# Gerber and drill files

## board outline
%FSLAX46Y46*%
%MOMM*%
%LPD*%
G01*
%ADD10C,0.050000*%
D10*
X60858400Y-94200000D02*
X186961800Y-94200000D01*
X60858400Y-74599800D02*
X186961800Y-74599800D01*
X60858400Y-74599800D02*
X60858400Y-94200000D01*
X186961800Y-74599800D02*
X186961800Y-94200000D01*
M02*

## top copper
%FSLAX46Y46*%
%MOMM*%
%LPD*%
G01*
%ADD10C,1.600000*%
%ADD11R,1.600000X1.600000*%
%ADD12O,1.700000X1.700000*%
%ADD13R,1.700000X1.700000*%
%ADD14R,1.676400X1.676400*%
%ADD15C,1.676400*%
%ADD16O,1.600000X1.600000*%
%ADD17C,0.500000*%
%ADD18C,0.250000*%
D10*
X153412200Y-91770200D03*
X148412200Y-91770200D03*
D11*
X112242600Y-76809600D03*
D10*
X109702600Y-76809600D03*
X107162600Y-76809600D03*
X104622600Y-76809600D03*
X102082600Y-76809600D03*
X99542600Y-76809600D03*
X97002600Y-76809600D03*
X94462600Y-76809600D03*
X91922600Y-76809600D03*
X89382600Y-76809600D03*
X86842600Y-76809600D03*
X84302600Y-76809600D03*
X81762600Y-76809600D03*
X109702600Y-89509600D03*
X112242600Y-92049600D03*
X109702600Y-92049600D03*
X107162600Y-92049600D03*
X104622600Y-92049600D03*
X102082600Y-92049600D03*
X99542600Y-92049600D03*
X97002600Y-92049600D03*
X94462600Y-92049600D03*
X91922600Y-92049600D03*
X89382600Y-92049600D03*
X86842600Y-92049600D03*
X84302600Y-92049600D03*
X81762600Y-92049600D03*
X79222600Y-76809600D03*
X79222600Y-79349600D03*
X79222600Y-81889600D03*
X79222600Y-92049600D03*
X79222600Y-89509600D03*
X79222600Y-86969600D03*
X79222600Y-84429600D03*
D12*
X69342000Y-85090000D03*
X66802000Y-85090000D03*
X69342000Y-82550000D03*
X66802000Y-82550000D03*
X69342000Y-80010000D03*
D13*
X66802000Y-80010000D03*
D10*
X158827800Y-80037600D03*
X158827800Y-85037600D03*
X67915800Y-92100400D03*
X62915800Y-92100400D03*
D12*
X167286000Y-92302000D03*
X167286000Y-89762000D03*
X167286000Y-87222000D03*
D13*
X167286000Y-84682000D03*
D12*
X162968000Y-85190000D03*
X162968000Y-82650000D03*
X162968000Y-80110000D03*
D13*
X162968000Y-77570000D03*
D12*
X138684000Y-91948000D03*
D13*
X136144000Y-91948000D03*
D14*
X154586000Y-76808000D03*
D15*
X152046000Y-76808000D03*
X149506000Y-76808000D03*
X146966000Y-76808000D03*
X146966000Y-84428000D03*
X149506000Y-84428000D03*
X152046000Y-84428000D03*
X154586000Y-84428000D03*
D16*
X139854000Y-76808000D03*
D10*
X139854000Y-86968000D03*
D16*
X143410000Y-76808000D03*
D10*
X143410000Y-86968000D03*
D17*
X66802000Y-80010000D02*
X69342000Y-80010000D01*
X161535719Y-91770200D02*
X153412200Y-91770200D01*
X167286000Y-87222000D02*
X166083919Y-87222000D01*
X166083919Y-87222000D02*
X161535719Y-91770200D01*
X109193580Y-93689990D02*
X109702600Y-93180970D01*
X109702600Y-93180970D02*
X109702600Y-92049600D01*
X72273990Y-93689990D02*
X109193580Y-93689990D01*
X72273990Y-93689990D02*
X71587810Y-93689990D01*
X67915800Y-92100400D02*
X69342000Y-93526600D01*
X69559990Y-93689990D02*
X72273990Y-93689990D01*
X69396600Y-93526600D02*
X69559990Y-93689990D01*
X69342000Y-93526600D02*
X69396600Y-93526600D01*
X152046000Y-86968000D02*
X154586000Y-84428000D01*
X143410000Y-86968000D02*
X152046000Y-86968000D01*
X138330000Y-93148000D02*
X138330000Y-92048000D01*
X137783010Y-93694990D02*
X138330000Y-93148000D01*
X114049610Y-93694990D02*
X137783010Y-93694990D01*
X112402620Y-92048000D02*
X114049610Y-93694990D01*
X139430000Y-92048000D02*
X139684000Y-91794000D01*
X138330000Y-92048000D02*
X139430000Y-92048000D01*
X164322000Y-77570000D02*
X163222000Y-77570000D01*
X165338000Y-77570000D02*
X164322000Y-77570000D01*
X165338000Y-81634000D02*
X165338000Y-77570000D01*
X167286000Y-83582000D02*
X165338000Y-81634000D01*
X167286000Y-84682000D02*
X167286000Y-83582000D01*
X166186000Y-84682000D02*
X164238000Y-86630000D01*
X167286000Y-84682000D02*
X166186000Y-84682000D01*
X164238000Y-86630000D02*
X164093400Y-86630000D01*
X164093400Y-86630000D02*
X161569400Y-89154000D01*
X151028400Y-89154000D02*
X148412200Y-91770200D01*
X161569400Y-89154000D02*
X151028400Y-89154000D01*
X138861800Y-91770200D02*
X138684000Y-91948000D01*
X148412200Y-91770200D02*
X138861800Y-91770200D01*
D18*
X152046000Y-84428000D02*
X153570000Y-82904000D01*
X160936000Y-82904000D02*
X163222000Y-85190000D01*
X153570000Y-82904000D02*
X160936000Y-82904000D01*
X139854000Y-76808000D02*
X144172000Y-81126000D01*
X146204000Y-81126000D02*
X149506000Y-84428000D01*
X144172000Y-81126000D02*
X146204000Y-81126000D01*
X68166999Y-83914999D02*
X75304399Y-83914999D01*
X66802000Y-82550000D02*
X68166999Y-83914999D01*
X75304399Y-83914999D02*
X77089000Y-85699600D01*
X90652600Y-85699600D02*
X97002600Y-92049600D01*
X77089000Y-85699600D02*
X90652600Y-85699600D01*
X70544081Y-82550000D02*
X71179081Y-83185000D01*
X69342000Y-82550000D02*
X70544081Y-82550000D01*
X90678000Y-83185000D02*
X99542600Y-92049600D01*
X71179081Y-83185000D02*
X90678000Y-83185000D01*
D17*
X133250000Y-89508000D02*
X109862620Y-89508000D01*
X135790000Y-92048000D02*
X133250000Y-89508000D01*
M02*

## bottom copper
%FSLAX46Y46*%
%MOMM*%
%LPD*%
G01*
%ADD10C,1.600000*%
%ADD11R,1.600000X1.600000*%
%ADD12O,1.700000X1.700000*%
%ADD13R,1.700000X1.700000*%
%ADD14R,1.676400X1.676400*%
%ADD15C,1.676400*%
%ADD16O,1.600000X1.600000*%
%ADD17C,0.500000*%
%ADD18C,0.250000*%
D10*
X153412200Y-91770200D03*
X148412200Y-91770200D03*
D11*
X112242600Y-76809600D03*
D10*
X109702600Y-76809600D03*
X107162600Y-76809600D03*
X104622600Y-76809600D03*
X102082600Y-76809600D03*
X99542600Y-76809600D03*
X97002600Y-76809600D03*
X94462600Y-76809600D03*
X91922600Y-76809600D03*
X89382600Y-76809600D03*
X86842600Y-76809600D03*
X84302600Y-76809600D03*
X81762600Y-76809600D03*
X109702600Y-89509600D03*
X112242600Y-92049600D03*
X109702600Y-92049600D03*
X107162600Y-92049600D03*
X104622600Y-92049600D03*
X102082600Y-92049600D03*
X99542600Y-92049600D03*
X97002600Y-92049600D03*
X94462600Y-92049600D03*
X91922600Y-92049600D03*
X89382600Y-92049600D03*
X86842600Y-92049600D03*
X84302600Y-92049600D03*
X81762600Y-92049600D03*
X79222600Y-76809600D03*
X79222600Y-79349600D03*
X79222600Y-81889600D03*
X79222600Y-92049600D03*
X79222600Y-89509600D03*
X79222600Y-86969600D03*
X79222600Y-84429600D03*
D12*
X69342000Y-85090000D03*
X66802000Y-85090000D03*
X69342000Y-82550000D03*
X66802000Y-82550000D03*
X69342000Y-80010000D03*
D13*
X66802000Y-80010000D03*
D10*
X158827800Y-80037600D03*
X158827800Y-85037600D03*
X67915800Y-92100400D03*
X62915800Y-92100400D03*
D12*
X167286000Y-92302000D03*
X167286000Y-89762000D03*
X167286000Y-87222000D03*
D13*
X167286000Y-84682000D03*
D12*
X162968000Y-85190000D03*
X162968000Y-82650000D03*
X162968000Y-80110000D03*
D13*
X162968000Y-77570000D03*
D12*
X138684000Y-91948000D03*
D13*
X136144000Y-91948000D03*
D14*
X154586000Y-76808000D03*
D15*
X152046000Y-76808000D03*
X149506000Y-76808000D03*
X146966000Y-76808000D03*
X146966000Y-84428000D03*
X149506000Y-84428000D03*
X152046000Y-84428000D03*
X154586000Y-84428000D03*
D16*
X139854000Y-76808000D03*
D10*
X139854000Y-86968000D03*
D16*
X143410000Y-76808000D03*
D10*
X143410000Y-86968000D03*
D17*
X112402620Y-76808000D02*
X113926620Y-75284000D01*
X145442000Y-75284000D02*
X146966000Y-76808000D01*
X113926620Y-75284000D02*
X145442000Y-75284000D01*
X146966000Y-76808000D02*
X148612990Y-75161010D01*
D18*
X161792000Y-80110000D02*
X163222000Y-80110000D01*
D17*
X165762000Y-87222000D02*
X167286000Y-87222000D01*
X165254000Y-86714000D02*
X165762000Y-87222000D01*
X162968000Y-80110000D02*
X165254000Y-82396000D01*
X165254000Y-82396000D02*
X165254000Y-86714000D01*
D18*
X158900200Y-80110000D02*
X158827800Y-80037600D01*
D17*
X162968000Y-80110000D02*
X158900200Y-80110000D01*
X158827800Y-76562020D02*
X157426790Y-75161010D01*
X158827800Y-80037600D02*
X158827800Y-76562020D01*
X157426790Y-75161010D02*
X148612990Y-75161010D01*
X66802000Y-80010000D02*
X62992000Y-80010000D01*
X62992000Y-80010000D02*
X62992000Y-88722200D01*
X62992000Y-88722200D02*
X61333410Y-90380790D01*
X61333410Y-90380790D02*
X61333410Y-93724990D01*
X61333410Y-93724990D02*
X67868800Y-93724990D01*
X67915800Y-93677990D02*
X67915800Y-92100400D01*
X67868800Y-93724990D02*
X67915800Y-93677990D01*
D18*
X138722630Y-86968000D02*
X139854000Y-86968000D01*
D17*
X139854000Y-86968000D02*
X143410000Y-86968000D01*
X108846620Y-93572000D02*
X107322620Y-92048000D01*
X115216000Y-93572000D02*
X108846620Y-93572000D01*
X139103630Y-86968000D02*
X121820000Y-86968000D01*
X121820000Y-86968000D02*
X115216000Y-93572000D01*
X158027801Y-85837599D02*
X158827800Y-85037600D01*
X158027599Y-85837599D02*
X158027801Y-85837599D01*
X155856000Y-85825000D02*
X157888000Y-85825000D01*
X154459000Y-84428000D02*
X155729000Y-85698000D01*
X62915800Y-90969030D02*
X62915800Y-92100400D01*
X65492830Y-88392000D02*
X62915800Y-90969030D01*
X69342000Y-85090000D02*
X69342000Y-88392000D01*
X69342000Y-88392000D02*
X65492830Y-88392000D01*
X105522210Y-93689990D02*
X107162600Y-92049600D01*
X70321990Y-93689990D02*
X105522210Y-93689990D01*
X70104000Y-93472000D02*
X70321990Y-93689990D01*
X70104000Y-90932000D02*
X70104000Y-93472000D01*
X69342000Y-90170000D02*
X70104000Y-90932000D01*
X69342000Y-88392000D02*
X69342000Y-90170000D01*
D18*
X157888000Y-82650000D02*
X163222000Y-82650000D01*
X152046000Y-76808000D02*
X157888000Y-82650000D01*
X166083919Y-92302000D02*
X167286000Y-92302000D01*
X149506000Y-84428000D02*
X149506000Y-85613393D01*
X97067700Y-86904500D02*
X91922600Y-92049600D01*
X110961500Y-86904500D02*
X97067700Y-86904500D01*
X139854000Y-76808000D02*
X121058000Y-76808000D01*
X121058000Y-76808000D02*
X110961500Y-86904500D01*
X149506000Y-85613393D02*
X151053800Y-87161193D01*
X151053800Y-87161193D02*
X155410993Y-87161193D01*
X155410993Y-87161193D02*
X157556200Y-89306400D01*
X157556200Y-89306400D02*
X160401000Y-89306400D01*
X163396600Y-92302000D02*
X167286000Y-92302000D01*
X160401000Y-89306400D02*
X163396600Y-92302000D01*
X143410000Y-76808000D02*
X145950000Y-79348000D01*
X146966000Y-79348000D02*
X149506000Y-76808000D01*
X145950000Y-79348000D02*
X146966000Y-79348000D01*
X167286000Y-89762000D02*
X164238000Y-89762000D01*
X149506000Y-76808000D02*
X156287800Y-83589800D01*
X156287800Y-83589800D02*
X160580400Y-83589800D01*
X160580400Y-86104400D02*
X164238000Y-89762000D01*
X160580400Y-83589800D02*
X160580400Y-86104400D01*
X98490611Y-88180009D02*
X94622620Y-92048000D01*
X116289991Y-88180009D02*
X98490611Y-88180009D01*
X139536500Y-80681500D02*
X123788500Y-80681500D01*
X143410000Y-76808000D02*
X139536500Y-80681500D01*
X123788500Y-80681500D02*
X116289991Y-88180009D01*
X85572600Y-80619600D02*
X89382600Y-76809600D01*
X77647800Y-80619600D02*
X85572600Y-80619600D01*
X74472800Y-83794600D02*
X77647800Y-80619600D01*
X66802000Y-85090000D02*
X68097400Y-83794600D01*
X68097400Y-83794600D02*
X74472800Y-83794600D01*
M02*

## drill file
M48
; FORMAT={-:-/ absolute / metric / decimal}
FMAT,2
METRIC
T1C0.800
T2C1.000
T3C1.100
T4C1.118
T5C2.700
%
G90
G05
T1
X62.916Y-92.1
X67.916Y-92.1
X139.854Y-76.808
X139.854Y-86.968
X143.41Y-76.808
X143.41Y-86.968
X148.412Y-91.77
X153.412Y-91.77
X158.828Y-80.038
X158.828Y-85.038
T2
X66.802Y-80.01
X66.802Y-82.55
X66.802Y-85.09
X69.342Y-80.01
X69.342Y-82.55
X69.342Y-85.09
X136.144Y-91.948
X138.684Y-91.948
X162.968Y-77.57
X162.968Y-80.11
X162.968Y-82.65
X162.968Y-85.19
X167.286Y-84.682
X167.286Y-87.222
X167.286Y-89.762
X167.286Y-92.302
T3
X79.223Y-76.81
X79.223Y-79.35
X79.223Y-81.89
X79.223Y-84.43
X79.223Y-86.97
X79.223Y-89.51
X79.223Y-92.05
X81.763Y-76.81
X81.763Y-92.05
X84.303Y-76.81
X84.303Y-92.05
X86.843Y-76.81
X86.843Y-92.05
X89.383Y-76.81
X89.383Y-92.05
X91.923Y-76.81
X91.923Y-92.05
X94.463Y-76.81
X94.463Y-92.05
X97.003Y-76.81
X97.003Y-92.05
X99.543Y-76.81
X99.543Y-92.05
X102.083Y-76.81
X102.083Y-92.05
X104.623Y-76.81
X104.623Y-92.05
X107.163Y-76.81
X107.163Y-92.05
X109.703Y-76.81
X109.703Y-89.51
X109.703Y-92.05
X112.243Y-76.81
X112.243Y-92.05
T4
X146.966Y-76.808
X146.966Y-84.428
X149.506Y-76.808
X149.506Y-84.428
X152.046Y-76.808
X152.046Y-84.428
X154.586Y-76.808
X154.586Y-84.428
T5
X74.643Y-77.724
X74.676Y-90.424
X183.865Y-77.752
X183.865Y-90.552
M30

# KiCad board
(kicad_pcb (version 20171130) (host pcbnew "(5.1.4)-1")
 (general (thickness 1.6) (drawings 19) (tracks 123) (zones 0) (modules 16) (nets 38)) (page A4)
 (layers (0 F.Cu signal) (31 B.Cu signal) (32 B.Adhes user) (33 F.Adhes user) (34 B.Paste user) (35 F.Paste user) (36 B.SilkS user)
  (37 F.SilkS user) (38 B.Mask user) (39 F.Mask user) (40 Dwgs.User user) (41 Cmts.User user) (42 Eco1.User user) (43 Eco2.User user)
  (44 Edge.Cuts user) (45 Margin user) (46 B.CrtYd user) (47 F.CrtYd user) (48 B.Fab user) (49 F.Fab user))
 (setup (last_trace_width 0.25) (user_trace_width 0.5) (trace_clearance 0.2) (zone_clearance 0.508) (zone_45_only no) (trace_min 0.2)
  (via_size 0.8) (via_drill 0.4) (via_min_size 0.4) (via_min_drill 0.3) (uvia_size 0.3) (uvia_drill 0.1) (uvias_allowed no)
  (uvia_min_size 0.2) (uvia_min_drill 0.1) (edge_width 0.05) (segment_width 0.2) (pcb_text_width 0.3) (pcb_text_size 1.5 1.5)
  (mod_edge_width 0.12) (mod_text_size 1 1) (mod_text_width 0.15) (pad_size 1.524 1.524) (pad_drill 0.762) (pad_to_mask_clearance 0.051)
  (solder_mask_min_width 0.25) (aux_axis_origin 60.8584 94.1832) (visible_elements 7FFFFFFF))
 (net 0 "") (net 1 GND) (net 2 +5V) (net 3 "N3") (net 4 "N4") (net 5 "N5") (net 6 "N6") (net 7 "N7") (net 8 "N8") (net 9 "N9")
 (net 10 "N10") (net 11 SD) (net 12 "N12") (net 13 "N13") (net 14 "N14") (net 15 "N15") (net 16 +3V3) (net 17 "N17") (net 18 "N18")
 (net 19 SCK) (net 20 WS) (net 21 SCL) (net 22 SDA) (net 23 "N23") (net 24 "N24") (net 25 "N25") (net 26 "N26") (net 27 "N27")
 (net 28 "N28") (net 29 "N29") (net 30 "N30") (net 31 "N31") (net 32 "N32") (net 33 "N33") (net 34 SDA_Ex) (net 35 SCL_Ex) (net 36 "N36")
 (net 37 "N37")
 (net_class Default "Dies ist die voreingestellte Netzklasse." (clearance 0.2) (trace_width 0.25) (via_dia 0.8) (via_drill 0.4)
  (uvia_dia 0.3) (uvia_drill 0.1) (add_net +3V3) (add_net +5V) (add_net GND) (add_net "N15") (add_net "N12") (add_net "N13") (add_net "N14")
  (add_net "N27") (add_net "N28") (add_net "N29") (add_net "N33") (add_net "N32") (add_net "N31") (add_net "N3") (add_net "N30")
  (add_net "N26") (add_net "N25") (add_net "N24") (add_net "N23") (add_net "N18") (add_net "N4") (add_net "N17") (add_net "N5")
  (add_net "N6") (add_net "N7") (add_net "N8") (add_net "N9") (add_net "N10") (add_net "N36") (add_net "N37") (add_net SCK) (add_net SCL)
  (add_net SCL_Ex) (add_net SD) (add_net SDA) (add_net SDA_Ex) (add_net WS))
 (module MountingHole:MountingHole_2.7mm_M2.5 (layer F.Cu) (at 74.676 90.424)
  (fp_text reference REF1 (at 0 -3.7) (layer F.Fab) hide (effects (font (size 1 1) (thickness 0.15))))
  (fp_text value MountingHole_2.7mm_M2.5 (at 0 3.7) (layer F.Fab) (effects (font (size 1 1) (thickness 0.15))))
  (pad 1 np_thru_hole circle (at 0 0) (size 2.7 2.7) (drill 2.7) (layers *.Cu *.Mask)))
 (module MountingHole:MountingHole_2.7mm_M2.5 (layer F.Cu) (at 74.643 77.724)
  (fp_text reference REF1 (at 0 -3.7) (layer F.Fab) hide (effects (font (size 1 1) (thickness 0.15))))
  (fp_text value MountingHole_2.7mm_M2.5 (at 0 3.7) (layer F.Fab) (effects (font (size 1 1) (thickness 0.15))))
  (pad 1 np_thru_hole circle (at 0 0) (size 2.7 2.7) (drill 2.7) (layers *.Cu *.Mask)))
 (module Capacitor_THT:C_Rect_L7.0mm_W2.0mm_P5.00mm (layer F.Cu) (at 148.4122 91.7702)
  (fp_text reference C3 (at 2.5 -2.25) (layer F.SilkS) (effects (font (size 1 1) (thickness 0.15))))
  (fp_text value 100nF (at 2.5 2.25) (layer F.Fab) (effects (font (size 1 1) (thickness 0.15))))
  (pad 2 thru_hole circle (at 5 0) (size 1.6 1.6) (drill 0.8) (layers *.Cu *.Mask) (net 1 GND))
  (pad 1 thru_hole circle (at 0 0) (size 1.6 1.6) (drill 0.8) (layers *.Cu *.Mask) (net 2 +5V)))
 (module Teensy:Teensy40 (layer F.Cu) (at 95.7326 84.4296 180)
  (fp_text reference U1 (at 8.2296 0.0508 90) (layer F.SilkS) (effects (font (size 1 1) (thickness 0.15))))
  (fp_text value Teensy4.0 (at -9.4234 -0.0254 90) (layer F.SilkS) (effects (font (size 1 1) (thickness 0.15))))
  (pad 1 thru_hole rect (at -16.51 7.62 180) (size 1.6 1.6) (drill 1.1) (layers *.Cu *.Mask) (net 1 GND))
  (pad 2 thru_hole circle (at -13.97 7.62 180) (size 1.6 1.6) (drill 1.1) (layers *.Cu *.Mask) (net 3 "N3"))
  (pad 3 thru_hole circle (at -11.43 7.62 180) (size 1.6 1.6) (drill 1.1) (layers *.Cu *.Mask) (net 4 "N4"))
  (pad 4 thru_hole circle (at -8.89 7.62 180) (size 1.6 1.6) (drill 1.1) (layers *.Cu *.Mask) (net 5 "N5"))
  (pad 5 thru_hole circle (at -6.35 7.62 180) (size 1.6 1.6) (drill 1.1) (layers *.Cu *.Mask) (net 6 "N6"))
  (pad 6 thru_hole circle (at -3.81 7.62 180) (size 1.6 1.6) (drill 1.1) (layers *.Cu *.Mask) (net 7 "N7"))
  (pad 7 thru_hole circle (at -1.27 7.62 180) (size 1.6 1.6) (drill 1.1) (layers *.Cu *.Mask) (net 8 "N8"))
  (pad 8 thru_hole circle (at 1.27 7.62 180) (size 1.6 1.6) (drill 1.1) (layers *.Cu *.Mask) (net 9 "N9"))
  (pad 9 thru_hole circle (at 3.81 7.62 180) (size 1.6 1.6) (drill 1.1) (layers *.Cu *.Mask) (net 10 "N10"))
  (pad 10 thru_hole circle (at 6.35 7.62 180) (size 1.6 1.6) (drill 1.1) (layers *.Cu *.Mask) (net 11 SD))
  (pad 11 thru_hole circle (at 8.89 7.62 180) (size 1.6 1.6) (drill 1.1) (layers *.Cu *.Mask) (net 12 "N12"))
  (pad 12 thru_hole circle (at 11.43 7.62 180) (size 1.6 1.6) (drill 1.1) (layers *.Cu *.Mask) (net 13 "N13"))
  (pad 13 thru_hole circle (at 13.97 7.62 180) (size 1.6 1.6) (drill 1.1) (layers *.Cu *.Mask) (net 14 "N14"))
  (pad 34 thru_hole circle (at -13.97 -5.08 180) (size 1.6 1.6) (drill 1.1) (layers *.Cu *.Mask) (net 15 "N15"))
  (pad 33 thru_hole circle (at -16.51 -7.62 180) (size 1.6 1.6) (drill 1.1) (layers *.Cu *.Mask) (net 2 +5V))
  (pad 32 thru_hole circle (at -13.97 -7.62 180) (size 1.6 1.6) (drill 1.1) (layers *.Cu *.Mask) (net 1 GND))
  (pad 31 thru_hole circle (at -11.43 -7.62 180) (size 1.6 1.6) (drill 1.1) (layers *.Cu *.Mask) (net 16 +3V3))
  (pad 30 thru_hole circle (at -8.89 -7.62 180) (size 1.6 1.6) (drill 1.1) (layers *.Cu *.Mask) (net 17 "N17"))
  (pad 29 thru_hole circle (at -6.35 -7.62 180) (size 1.6 1.6) (drill 1.1) (layers *.Cu *.Mask) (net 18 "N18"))
  (pad 28 thru_hole circle (at -3.81 -7.62 180) (size 1.6 1.6) (drill 1.1) (layers *.Cu *.Mask) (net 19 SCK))
  (pad 27 thru_hole circle (at -1.27 -7.62 180) (size 1.6 1.6) (drill 1.1) (layers *.Cu *.Mask) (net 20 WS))
  (pad 26 thru_hole circle (at 1.27 -7.62 180) (size 1.6 1.6) (drill 1.1) (layers *.Cu *.Mask) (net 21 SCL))
  (pad 25 thru_hole circle (at 3.81 -7.62 180) (size 1.6 1.6) (drill 1.1) (layers *.Cu *.Mask) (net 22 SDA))
  (pad 24 thru_hole circle (at 6.35 -7.62 180) (size 1.6 1.6) (drill 1.1) (layers *.Cu *.Mask) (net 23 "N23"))
  (pad 23 thru_hole circle (at 8.89 -7.62 180) (size 1.6 1.6) (drill 1.1) (layers *.Cu *.Mask) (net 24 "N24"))
  (pad 22 thru_hole circle (at 11.43 -7.62 180) (size 1.6 1.6) (drill 1.1) (layers *.Cu *.Mask) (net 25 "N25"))
  (pad 21 thru_hole circle (at 13.97 -7.62 180) (size 1.6 1.6) (drill 1.1) (layers *.Cu *.Mask) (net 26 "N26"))
  (pad 14 thru_hole circle (at 16.51 7.62 180) (size 1.6 1.6) (drill 1.1) (layers *.Cu *.Mask) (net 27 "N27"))
  (pad 15 thru_hole circle (at 16.51 5.08 180) (size 1.6 1.6) (drill 1.1) (layers *.Cu *.Mask) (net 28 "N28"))
  (pad 16 thru_hole circle (at 16.51 2.54 180) (size 1.6 1.6) (drill 1.1) (layers *.Cu *.Mask) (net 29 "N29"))
  (pad 20 thru_hole circle (at 16.51 -7.62 180) (size 1.6 1.6) (drill 1.1) (layers *.Cu *.Mask) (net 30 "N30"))
  (pad 19 thru_hole circle (at 16.51 -5.08 180) (size 1.6 1.6) (drill 1.1) (layers *.Cu *.Mask) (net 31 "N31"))
  (pad 18 thru_hole circle (at 16.51 -2.54 180) (size 1.6 1.6) (drill 1.1) (layers *.Cu *.Mask) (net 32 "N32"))
  (pad 17 thru_hole circle (at 16.51 0 180) (size 1.6 1.6) (drill 1.1) (layers *.Cu *.Mask) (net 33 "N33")))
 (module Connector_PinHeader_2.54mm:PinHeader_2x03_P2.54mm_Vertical (layer F.Cu) (at 66.802 80.01)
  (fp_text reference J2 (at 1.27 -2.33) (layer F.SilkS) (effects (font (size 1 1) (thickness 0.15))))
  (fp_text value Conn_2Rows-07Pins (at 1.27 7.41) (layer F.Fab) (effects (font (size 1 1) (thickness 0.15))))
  (pad 6 thru_hole oval (at 2.54 5.08) (size 1.7 1.7) (drill 1) (layers *.Cu *.Mask) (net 16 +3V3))
  (pad 5 thru_hole oval (at 0 5.08) (size 1.7 1.7) (drill 1) (layers *.Cu *.Mask) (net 11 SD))
  (pad 4 thru_hole oval (at 2.54 2.54) (size 1.7 1.7) (drill 1) (layers *.Cu *.Mask) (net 19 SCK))
  (pad 3 thru_hole oval (at 0 2.54) (size 1.7 1.7) (drill 1) (layers *.Cu *.Mask) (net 20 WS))
  (pad 2 thru_hole oval (at 2.54 0) (size 1.7 1.7) (drill 1) (layers *.Cu *.Mask) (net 1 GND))
  (pad 1 thru_hole rect (at 0 0) (size 1.7 1.7) (drill 1) (layers *.Cu *.Mask) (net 1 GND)))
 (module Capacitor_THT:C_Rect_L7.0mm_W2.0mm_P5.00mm (layer F.Cu) (at 158.8278 85.0376 90)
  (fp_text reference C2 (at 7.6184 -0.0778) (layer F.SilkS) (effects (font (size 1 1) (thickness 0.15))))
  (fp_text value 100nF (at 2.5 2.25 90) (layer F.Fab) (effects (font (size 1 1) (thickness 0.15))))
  (pad 2 thru_hole circle (at 5 0 90) (size 1.6 1.6) (drill 0.8) (layers *.Cu *.Mask) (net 1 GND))
  (pad 1 thru_hole circle (at 0 0 90) (size 1.6 1.6) (drill 0.8) (layers *.Cu *.Mask) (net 16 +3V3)))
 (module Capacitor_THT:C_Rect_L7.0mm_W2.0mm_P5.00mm (layer F.Cu) (at 62.9158 92.1004)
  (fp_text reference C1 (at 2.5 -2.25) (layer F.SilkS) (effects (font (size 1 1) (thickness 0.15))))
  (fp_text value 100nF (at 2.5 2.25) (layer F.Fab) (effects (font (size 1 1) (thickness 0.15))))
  (pad 2 thru_hole circle (at 5 0) (size 1.6 1.6) (drill 0.8) (layers *.Cu *.Mask) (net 1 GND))
  (pad 1 thru_hole circle (at 0 0) (size 1.6 1.6) (drill 0.8) (layers *.Cu *.Mask) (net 16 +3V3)))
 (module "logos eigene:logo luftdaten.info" (layer F.Cu) (at 121.4898 88.6698)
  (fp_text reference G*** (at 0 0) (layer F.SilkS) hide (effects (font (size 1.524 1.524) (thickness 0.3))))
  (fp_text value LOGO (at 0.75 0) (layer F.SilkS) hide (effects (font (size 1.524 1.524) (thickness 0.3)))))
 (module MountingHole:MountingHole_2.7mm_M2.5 (layer F.Cu) (at 183.8654 90.5524)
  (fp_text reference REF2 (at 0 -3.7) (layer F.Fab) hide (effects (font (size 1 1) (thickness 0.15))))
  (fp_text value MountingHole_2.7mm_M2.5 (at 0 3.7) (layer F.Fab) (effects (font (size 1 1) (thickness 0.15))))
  (pad 1 np_thru_hole circle (at 0 0) (size 2.7 2.7) (drill 2.7) (layers *.Cu *.Mask)))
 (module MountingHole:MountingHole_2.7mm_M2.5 (layer F.Cu) (at 183.8654 77.7518)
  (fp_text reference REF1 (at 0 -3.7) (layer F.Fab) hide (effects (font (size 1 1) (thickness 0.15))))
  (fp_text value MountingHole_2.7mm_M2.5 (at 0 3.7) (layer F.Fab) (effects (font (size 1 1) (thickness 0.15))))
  (pad 1 np_thru_hole circle (at 0 0) (size 2.7 2.7) (drill 2.7) (layers *.Cu *.Mask)))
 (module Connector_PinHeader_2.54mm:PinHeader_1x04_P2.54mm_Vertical (layer F.Cu) (at 167.286 84.682)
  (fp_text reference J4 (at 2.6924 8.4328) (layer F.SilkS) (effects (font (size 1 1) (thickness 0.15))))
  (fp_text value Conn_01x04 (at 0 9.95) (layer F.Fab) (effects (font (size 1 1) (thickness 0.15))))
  (pad 4 thru_hole oval (at 0 7.62) (size 1.7 1.7) (drill 1) (layers *.Cu *.Mask) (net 22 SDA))
  (pad 3 thru_hole oval (at 0 5.08) (size 1.7 1.7) (drill 1) (layers *.Cu *.Mask) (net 21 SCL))
  (pad 2 thru_hole oval (at 0 2.54) (size 1.7 1.7) (drill 1) (layers *.Cu *.Mask) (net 1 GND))
  (pad 1 thru_hole rect (at 0 0) (size 1.7 1.7) (drill 1) (layers *.Cu *.Mask) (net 2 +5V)))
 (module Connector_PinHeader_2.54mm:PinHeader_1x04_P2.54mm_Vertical (layer F.Cu) (at 162.968 77.57)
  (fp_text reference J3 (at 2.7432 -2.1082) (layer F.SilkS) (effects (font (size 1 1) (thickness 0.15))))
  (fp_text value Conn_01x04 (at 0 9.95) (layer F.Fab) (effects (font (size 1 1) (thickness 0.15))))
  (pad 4 thru_hole oval (at 0 7.62) (size 1.7 1.7) (drill 1) (layers *.Cu *.Mask) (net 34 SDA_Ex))
  (pad 3 thru_hole oval (at 0 5.08) (size 1.7 1.7) (drill 1) (layers *.Cu *.Mask) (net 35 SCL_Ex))
  (pad 2 thru_hole oval (at 0 2.54) (size 1.7 1.7) (drill 1) (layers *.Cu *.Mask) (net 1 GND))
  (pad 1 thru_hole rect (at 0 0) (size 1.7 1.7) (drill 1) (layers *.Cu *.Mask) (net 2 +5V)))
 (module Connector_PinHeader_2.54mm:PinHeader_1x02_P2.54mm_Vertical (layer F.Cu) (at 136.144 91.948 90)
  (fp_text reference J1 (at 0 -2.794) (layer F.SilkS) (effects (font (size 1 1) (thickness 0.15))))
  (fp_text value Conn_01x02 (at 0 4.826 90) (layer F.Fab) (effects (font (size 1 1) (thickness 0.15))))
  (pad 2 thru_hole oval (at 0 2.54 90) (size 1.7 1.7) (drill 1) (layers *.Cu *.Mask) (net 2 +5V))
  (pad 1 thru_hole rect (at 0 0 90) (size 1.7 1.7) (drill 1) (layers *.Cu *.Mask) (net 15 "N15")))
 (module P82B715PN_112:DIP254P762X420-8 (layer F.Cu) (at 146.966 84.428 270)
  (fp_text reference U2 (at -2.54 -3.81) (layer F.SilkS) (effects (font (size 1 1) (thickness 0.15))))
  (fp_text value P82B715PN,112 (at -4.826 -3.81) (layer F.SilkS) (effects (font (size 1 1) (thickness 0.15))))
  (pad 1 thru_hole rect (at -7.62 -7.62 270) (size 1.6764 1.6764) (drill 1.1176) (layers *.Cu *.Mask) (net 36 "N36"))
  (pad 2 thru_hole circle (at -7.62 -5.08 270) (size 1.6764 1.6764) (drill 1.1176) (layers *.Cu *.Mask) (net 35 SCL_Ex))
  (pad 3 thru_hole circle (at -7.62 -2.54 270) (size 1.6764 1.6764) (drill 1.1176) (layers *.Cu *.Mask) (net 21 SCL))
  (pad 4 thru_hole circle (at -7.62 0 270) (size 1.6764 1.6764) (drill 1.1176) (layers *.Cu *.Mask) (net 1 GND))
  (pad 5 thru_hole circle (at 0 0 270) (size 1.6764 1.6764) (drill 1.1176) (layers *.Cu *.Mask) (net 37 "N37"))
  (pad 6 thru_hole circle (at 0 -2.54 270) (size 1.6764 1.6764) (drill 1.1176) (layers *.Cu *.Mask) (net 22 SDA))
  (pad 7 thru_hole circle (at 0 -5.08 270) (size 1.6764 1.6764) (drill 1.1176) (layers *.Cu *.Mask) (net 34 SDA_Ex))
  (pad 8 thru_hole circle (at 0 -7.62 270) (size 1.6764 1.6764) (drill 1.1176) (layers *.Cu *.Mask) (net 16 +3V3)))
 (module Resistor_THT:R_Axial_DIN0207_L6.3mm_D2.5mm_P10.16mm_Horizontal (layer F.Cu) (at 139.854 86.968 90)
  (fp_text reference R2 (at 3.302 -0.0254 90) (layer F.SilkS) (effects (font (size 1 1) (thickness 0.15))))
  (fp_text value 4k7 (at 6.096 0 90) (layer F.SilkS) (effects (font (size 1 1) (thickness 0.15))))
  (pad 2 thru_hole oval (at 10.16 0 90) (size 1.6 1.6) (drill 0.8) (layers *.Cu *.Mask) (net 22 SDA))
  (pad 1 thru_hole circle (at 0 0 90) (size 1.6 1.6) (drill 0.8) (layers *.Cu *.Mask) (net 16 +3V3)))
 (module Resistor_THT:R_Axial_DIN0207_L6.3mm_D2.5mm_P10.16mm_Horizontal (layer F.Cu) (at 143.41 86.968 90)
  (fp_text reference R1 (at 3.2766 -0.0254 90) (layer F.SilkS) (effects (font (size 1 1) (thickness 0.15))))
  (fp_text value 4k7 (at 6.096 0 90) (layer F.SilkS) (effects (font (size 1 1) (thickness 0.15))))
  (pad 2 thru_hole oval (at 10.16 0 90) (size 1.6 1.6) (drill 0.8) (layers *.Cu *.Mask) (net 21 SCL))
  (pad 1 thru_hole circle (at 0 0 90) (size 1.6 1.6) (drill 0.8) (layers *.Cu *.Mask) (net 16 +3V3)))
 (gr_line (start 60.8584 94.2) (end 186.9618 94.2) (layer Edge.Cuts) (width 0.05))
 (gr_line (start 60.8584 74.5998) (end 186.9618 74.5998) (layer Edge.Cuts) (width 0.05))
 (gr_line (start 60.8584 74.5998) (end 60.8584 94.2) (layer Edge.Cuts) (width 0.05))
 (gr_line (start 186.9618 74.5998) (end 186.9618 94.2) (layer Edge.Cuts) (width 0.05))
 (segment (start 112.40262 76.808) (end 113.92662 75.284) (width 0.5) (layer B.Cu) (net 1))
 (segment (start 145.442 75.284) (end 146.966 76.808) (width 0.5) (layer B.Cu) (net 1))
 (segment (start 113.92662 75.284) (end 145.442 75.284) (width 0.5) (layer B.Cu) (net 1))
 (segment (start 146.966 76.808) (end 148.61299 75.16101) (width 0.5) (layer B.Cu) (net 1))
 (segment (start 161.792 80.11) (end 163.222 80.11) (width 0.25) (layer B.Cu) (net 1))
 (segment (start 165.762 87.222) (end 167.286 87.222) (width 0.5) (layer B.Cu) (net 1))
 (segment (start 165.254 86.714) (end 165.762 87.222) (width 0.5) (layer B.Cu) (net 1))
 (segment (start 162.968 80.11) (end 165.254 82.396) (width 0.5) (layer B.Cu) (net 1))
 (segment (start 165.254 82.396) (end 165.254 86.714) (width 0.5) (layer B.Cu) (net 1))
 (segment (start 158.9002 80.11) (end 158.8278 80.0376) (width 0.25) (layer B.Cu) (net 1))
 (segment (start 162.968 80.11) (end 158.9002 80.11) (width 0.5) (layer B.Cu) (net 1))
 (segment (start 158.8278 76.56202) (end 157.42679 75.16101) (width 0.5) (layer B.Cu) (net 1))
 (segment (start 158.8278 80.0376) (end 158.8278 76.56202) (width 0.5) (layer B.Cu) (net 1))
 (segment (start 157.42679 75.16101) (end 148.61299 75.16101) (width 0.5) (layer B.Cu) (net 1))
 (segment (start 66.802 80.01) (end 69.342 80.01) (width 0.5) (layer F.Cu) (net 1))
 (segment (start 66.802 80.01) (end 62.992 80.01) (width 0.5) (layer B.Cu) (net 1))
 (segment (start 161.535719 91.7702) (end 153.4122 91.7702) (width 0.5) (layer F.Cu) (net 1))
 (segment (start 167.286 87.222) (end 166.083919 87.222) (width 0.5) (layer F.Cu) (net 1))
 (segment (start 166.083919 87.222) (end 161.535719 91.7702) (width 0.5) (layer F.Cu) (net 1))
 (segment (start 62.992 80.01) (end 62.992 88.7222) (width 0.5) (layer B.Cu) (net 1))
 (segment (start 62.992 88.7222) (end 61.33341 90.38079) (width 0.5) (layer B.Cu) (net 1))
 (segment (start 61.33341 90.38079) (end 61.33341 93.72499) (width 0.5) (layer B.Cu) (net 1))
 (segment (start 61.33341 93.72499) (end 67.8688 93.72499) (width 0.5) (layer B.Cu) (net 1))
 (segment (start 67.9158 93.67799) (end 67.9158 92.1004) (width 0.5) (layer B.Cu) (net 1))
 (segment (start 67.8688 93.72499) (end 67.9158 93.67799) (width 0.5) (layer B.Cu) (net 1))
 (segment (start 109.19358 93.68999) (end 109.7026 93.18097) (width 0.5) (layer F.Cu) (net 1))
 (segment (start 109.7026 93.18097) (end 109.7026 92.0496) (width 0.5) (layer F.Cu) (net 1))
 (segment (start 72.27399 93.68999) (end 109.19358 93.68999) (width 0.5) (layer F.Cu) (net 1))
 (segment (start 72.27399 93.68999) (end 71.58781 93.68999) (width 0.5) (layer F.Cu) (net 1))
 (segment (start 67.9158 92.1004) (end 69.342 93.5266) (width 0.5) (layer F.Cu) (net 1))
 (segment (start 69.55999 93.68999) (end 72.27399 93.68999) (width 0.5) (layer F.Cu) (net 1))
 (segment (start 69.3966 93.5266) (end 69.55999 93.68999) (width 0.5) (layer F.Cu) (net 1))
 (segment (start 69.342 93.5266) (end 69.3966 93.5266) (width 0.5) (layer F.Cu) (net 1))
 (segment (start 138.72263 86.968) (end 139.854 86.968) (width 0.25) (layer B.Cu) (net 16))
 (segment (start 139.854 86.968) (end 143.41 86.968) (width 0.5) (layer B.Cu) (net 16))
 (segment (start 152.046 86.968) (end 154.586 84.428) (width 0.5) (layer F.Cu) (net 16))
 (segment (start 143.41 86.968) (end 152.046 86.968) (width 0.5) (layer F.Cu) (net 16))
 (segment (start 108.84662 93.572) (end 107.32262 92.048) (width 0.5) (layer B.Cu) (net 16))
 (segment (start 115.216 93.572) (end 108.84662 93.572) (width 0.5) (layer B.Cu) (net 16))
 (segment (start 139.10363 86.968) (end 121.82 86.968) (width 0.5) (layer B.Cu) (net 16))
 (segment (start 121.82 86.968) (end 115.216 93.572) (width 0.5) (layer B.Cu) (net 16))
 (segment (start 158.027801 85.837599) (end 158.8278 85.0376) (width 0.5) (layer B.Cu) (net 16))
 (segment (start 158.027599 85.837599) (end 158.027801 85.837599) (width 0.5) (layer B.Cu) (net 16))
 (segment (start 155.856 85.825) (end 157.888 85.825) (width 0.5) (layer B.Cu) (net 16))
 (segment (start 154.459 84.428) (end 155.729 85.698) (width 0.5) (layer B.Cu) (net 16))
 (segment (start 62.9158 90.96903) (end 62.9158 92.1004) (width 0.5) (layer B.Cu) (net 16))
 (segment (start 65.49283 88.392) (end 62.9158 90.96903) (width 0.5) (layer B.Cu) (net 16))
 (segment (start 69.342 85.09) (end 69.342 88.392) (width 0.5) (layer B.Cu) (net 16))
 (segment (start 69.342 88.392) (end 65.49283 88.392) (width 0.5) (layer B.Cu) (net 16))
 (segment (start 105.52221 93.68999) (end 107.1626 92.0496) (width 0.5) (layer B.Cu) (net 16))
 (segment (start 70.32199 93.68999) (end 105.52221 93.68999) (width 0.5) (layer B.Cu) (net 16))
 (segment (start 70.104 93.472) (end 70.32199 93.68999) (width 0.5) (layer B.Cu) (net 16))
 (segment (start 70.104 90.932) (end 70.104 93.472) (width 0.5) (layer B.Cu) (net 16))
 (segment (start 69.342 90.17) (end 70.104 90.932) (width 0.5) (layer B.Cu) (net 16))
 (segment (start 69.342 88.392) (end 69.342 90.17) (width 0.5) (layer B.Cu) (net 16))
 (segment (start 138.33 93.148) (end 138.33 92.048) (width 0.5) (layer F.Cu) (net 2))
 (segment (start 137.78301 93.69499) (end 138.33 93.148) (width 0.5) (layer F.Cu) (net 2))
 (segment (start 114.04961 93.69499) (end 137.78301 93.69499) (width 0.5) (layer F.Cu) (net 2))
 (segment (start 112.40262 92.048) (end 114.04961 93.69499) (width 0.5) (layer F.Cu) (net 2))
 (segment (start 139.43 92.048) (end 139.684 91.794) (width 0.5) (layer F.Cu) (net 2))
 (segment (start 138.33 92.048) (end 139.43 92.048) (width 0.5) (layer F.Cu) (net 2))
 (segment (start 164.322 77.57) (end 163.222 77.57) (width 0.5) (layer F.Cu) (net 2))
 (segment (start 165.338 77.57) (end 164.322 77.57) (width 0.5) (layer F.Cu) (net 2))
 (segment (start 165.338 81.634) (end 165.338 77.57) (width 0.5) (layer F.Cu) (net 2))
 (segment (start 167.286 83.582) (end 165.338 81.634) (width 0.5) (layer F.Cu) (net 2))
 (segment (start 167.286 84.682) (end 167.286 83.582) (width 0.5) (layer F.Cu) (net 2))
 (segment (start 166.186 84.682) (end 164.238 86.63) (width 0.5) (layer F.Cu) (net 2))
 (segment (start 167.286 84.682) (end 166.186 84.682) (width 0.5) (layer F.Cu) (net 2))
 (segment (start 164.238 86.63) (end 164.0934 86.63) (width 0.5) (layer F.Cu) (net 2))
 (segment (start 164.0934 86.63) (end 161.5694 89.154) (width 0.5) (layer F.Cu) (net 2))
 (segment (start 151.0284 89.154) (end 148.4122 91.7702) (width 0.5) (layer F.Cu) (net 2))
 (segment (start 161.5694 89.154) (end 151.0284 89.154) (width 0.5) (layer F.Cu) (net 2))
 (segment (start 138.8618 91.7702) (end 138.684 91.948) (width 0.5) (layer F.Cu) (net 2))
 (segment (start 148.4122 91.7702) (end 138.8618 91.7702) (width 0.5) (layer F.Cu) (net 2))
 (segment (start 152.046 84.428) (end 153.57 82.904) (width 0.25) (layer F.Cu) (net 34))
 (segment (start 160.936 82.904) (end 163.222 85.19) (width 0.25) (layer F.Cu) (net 34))
 (segment (start 153.57 82.904) (end 160.936 82.904) (width 0.25) (layer F.Cu) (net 34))
 (segment (start 157.888 82.65) (end 163.222 82.65) (width 0.25) (layer B.Cu) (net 35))
 (segment (start 152.046 76.808) (end 157.888 82.65) (width 0.25) (layer B.Cu) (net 35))
 (segment (start 139.854 76.808) (end 144.172 81.126) (width 0.25) (layer F.Cu) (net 22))
 (segment (start 146.204 81.126) (end 149.506 84.428) (width 0.25) (layer F.Cu) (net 22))
 (segment (start 144.172 81.126) (end 146.204 81.126) (width 0.25) (layer F.Cu) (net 22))
 (segment (start 166.083919 92.302) (end 167.286 92.302) (width 0.25) (layer B.Cu) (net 22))
 (segment (start 149.506 84.428) (end 149.506 85.613393) (width 0.25) (layer B.Cu) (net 22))
 (segment (start 97.0677 86.9045) (end 91.9226 92.0496) (width 0.25) (layer B.Cu) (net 22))
 (segment (start 110.9615 86.9045) (end 97.0677 86.9045) (width 0.25) (layer B.Cu) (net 22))
 (segment (start 139.854 76.808) (end 121.058 76.808) (width 0.25) (layer B.Cu) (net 22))
 (segment (start 121.058 76.808) (end 110.9615 86.9045) (width 0.25) (layer B.Cu) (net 22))
 (segment (start 149.506 85.613393) (end 151.0538 87.161193) (width 0.25) (layer B.Cu) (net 22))
 (segment (start 151.0538 87.161193) (end 155.410993 87.161193) (width 0.25) (layer B.Cu) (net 22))
 (segment (start 155.410993 87.161193) (end 157.5562 89.3064) (width 0.25) (layer B.Cu) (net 22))
 (segment (start 157.5562 89.3064) (end 160.401 89.3064) (width 0.25) (layer B.Cu) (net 22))
 (segment (start 163.3966 92.302) (end 167.286 92.302) (width 0.25) (layer B.Cu) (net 22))
 (segment (start 160.401 89.3064) (end 163.3966 92.302) (width 0.25) (layer B.Cu) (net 22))
 (segment (start 143.41 76.808) (end 145.95 79.348) (width 0.25) (layer B.Cu) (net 21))
 (segment (start 146.966 79.348) (end 149.506 76.808) (width 0.25) (layer B.Cu) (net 21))
 (segment (start 145.95 79.348) (end 146.966 79.348) (width 0.25) (layer B.Cu) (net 21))
 (segment (start 167.286 89.762) (end 164.238 89.762) (width 0.25) (layer B.Cu) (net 21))
 (segment (start 149.506 76.808) (end 156.2878 83.5898) (width 0.25) (layer B.Cu) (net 21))
 (segment (start 156.2878 83.5898) (end 160.5804 83.5898) (width 0.25) (layer B.Cu) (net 21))
 (segment (start 160.5804 86.1044) (end 164.238 89.762) (width 0.25) (layer B.Cu) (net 21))
 (segment (start 160.5804 83.5898) (end 160.5804 86.1044) (width 0.25) (layer B.Cu) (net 21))
 (segment (start 98.490611 88.180009) (end 94.62262 92.048) (width 0.25) (layer B.Cu) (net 21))
 (segment (start 116.289991 88.180009) (end 98.490611 88.180009) (width 0.25) (layer B.Cu) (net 21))
 (segment (start 139.5365 80.6815) (end 123.7885 80.6815) (width 0.25) (layer B.Cu) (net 21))
 (segment (start 143.41 76.808) (end 139.5365 80.6815) (width 0.25) (layer B.Cu) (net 21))
 (segment (start 123.7885 80.6815) (end 116.289991 88.180009) (width 0.25) (layer B.Cu) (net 21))
 (segment (start 85.5726 80.6196) (end 89.3826 76.8096) (width 0.25) (layer B.Cu) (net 11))
 (segment (start 77.6478 80.6196) (end 85.5726 80.6196) (width 0.25) (layer B.Cu) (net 11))
 (segment (start 74.4728 83.7946) (end 77.6478 80.6196) (width 0.25) (layer B.Cu) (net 11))
 (segment (start 66.802 85.09) (end 68.0974 83.7946) (width 0.25) (layer B.Cu) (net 11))
 (segment (start 68.0974 83.7946) (end 74.4728 83.7946) (width 0.25) (layer B.Cu) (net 11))
 (segment (start 68.166999 83.914999) (end 75.304399 83.914999) (width 0.25) (layer F.Cu) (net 20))
 (segment (start 66.802 82.55) (end 68.166999 83.914999) (width 0.25) (layer F.Cu) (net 20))
 (segment (start 75.304399 83.914999) (end 77.089 85.6996) (width 0.25) (layer F.Cu) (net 20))
 (segment (start 90.6526 85.6996) (end 97.0026 92.0496) (width 0.25) (layer F.Cu) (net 20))
 (segment (start 77.089 85.6996) (end 90.6526 85.6996) (width 0.25) (layer F.Cu) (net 20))
 (segment (start 70.544081 82.55) (end 71.179081 83.185) (width 0.25) (layer F.Cu) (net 19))
 (segment (start 69.342 82.55) (end 70.544081 82.55) (width 0.25) (layer F.Cu) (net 19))
 (segment (start 90.678 83.185) (end 99.5426 92.0496) (width 0.25) (layer F.Cu) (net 19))
 (segment (start 71.179081 83.185) (end 90.678 83.185) (width 0.25) (layer F.Cu) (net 19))
 (segment (start 133.25 89.508) (end 109.86262 89.508) (width 0.5) (layer F.Cu) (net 15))
 (segment (start 135.79 92.048) (end 133.25 89.508) (width 0.5) (layer F.Cu) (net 15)))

